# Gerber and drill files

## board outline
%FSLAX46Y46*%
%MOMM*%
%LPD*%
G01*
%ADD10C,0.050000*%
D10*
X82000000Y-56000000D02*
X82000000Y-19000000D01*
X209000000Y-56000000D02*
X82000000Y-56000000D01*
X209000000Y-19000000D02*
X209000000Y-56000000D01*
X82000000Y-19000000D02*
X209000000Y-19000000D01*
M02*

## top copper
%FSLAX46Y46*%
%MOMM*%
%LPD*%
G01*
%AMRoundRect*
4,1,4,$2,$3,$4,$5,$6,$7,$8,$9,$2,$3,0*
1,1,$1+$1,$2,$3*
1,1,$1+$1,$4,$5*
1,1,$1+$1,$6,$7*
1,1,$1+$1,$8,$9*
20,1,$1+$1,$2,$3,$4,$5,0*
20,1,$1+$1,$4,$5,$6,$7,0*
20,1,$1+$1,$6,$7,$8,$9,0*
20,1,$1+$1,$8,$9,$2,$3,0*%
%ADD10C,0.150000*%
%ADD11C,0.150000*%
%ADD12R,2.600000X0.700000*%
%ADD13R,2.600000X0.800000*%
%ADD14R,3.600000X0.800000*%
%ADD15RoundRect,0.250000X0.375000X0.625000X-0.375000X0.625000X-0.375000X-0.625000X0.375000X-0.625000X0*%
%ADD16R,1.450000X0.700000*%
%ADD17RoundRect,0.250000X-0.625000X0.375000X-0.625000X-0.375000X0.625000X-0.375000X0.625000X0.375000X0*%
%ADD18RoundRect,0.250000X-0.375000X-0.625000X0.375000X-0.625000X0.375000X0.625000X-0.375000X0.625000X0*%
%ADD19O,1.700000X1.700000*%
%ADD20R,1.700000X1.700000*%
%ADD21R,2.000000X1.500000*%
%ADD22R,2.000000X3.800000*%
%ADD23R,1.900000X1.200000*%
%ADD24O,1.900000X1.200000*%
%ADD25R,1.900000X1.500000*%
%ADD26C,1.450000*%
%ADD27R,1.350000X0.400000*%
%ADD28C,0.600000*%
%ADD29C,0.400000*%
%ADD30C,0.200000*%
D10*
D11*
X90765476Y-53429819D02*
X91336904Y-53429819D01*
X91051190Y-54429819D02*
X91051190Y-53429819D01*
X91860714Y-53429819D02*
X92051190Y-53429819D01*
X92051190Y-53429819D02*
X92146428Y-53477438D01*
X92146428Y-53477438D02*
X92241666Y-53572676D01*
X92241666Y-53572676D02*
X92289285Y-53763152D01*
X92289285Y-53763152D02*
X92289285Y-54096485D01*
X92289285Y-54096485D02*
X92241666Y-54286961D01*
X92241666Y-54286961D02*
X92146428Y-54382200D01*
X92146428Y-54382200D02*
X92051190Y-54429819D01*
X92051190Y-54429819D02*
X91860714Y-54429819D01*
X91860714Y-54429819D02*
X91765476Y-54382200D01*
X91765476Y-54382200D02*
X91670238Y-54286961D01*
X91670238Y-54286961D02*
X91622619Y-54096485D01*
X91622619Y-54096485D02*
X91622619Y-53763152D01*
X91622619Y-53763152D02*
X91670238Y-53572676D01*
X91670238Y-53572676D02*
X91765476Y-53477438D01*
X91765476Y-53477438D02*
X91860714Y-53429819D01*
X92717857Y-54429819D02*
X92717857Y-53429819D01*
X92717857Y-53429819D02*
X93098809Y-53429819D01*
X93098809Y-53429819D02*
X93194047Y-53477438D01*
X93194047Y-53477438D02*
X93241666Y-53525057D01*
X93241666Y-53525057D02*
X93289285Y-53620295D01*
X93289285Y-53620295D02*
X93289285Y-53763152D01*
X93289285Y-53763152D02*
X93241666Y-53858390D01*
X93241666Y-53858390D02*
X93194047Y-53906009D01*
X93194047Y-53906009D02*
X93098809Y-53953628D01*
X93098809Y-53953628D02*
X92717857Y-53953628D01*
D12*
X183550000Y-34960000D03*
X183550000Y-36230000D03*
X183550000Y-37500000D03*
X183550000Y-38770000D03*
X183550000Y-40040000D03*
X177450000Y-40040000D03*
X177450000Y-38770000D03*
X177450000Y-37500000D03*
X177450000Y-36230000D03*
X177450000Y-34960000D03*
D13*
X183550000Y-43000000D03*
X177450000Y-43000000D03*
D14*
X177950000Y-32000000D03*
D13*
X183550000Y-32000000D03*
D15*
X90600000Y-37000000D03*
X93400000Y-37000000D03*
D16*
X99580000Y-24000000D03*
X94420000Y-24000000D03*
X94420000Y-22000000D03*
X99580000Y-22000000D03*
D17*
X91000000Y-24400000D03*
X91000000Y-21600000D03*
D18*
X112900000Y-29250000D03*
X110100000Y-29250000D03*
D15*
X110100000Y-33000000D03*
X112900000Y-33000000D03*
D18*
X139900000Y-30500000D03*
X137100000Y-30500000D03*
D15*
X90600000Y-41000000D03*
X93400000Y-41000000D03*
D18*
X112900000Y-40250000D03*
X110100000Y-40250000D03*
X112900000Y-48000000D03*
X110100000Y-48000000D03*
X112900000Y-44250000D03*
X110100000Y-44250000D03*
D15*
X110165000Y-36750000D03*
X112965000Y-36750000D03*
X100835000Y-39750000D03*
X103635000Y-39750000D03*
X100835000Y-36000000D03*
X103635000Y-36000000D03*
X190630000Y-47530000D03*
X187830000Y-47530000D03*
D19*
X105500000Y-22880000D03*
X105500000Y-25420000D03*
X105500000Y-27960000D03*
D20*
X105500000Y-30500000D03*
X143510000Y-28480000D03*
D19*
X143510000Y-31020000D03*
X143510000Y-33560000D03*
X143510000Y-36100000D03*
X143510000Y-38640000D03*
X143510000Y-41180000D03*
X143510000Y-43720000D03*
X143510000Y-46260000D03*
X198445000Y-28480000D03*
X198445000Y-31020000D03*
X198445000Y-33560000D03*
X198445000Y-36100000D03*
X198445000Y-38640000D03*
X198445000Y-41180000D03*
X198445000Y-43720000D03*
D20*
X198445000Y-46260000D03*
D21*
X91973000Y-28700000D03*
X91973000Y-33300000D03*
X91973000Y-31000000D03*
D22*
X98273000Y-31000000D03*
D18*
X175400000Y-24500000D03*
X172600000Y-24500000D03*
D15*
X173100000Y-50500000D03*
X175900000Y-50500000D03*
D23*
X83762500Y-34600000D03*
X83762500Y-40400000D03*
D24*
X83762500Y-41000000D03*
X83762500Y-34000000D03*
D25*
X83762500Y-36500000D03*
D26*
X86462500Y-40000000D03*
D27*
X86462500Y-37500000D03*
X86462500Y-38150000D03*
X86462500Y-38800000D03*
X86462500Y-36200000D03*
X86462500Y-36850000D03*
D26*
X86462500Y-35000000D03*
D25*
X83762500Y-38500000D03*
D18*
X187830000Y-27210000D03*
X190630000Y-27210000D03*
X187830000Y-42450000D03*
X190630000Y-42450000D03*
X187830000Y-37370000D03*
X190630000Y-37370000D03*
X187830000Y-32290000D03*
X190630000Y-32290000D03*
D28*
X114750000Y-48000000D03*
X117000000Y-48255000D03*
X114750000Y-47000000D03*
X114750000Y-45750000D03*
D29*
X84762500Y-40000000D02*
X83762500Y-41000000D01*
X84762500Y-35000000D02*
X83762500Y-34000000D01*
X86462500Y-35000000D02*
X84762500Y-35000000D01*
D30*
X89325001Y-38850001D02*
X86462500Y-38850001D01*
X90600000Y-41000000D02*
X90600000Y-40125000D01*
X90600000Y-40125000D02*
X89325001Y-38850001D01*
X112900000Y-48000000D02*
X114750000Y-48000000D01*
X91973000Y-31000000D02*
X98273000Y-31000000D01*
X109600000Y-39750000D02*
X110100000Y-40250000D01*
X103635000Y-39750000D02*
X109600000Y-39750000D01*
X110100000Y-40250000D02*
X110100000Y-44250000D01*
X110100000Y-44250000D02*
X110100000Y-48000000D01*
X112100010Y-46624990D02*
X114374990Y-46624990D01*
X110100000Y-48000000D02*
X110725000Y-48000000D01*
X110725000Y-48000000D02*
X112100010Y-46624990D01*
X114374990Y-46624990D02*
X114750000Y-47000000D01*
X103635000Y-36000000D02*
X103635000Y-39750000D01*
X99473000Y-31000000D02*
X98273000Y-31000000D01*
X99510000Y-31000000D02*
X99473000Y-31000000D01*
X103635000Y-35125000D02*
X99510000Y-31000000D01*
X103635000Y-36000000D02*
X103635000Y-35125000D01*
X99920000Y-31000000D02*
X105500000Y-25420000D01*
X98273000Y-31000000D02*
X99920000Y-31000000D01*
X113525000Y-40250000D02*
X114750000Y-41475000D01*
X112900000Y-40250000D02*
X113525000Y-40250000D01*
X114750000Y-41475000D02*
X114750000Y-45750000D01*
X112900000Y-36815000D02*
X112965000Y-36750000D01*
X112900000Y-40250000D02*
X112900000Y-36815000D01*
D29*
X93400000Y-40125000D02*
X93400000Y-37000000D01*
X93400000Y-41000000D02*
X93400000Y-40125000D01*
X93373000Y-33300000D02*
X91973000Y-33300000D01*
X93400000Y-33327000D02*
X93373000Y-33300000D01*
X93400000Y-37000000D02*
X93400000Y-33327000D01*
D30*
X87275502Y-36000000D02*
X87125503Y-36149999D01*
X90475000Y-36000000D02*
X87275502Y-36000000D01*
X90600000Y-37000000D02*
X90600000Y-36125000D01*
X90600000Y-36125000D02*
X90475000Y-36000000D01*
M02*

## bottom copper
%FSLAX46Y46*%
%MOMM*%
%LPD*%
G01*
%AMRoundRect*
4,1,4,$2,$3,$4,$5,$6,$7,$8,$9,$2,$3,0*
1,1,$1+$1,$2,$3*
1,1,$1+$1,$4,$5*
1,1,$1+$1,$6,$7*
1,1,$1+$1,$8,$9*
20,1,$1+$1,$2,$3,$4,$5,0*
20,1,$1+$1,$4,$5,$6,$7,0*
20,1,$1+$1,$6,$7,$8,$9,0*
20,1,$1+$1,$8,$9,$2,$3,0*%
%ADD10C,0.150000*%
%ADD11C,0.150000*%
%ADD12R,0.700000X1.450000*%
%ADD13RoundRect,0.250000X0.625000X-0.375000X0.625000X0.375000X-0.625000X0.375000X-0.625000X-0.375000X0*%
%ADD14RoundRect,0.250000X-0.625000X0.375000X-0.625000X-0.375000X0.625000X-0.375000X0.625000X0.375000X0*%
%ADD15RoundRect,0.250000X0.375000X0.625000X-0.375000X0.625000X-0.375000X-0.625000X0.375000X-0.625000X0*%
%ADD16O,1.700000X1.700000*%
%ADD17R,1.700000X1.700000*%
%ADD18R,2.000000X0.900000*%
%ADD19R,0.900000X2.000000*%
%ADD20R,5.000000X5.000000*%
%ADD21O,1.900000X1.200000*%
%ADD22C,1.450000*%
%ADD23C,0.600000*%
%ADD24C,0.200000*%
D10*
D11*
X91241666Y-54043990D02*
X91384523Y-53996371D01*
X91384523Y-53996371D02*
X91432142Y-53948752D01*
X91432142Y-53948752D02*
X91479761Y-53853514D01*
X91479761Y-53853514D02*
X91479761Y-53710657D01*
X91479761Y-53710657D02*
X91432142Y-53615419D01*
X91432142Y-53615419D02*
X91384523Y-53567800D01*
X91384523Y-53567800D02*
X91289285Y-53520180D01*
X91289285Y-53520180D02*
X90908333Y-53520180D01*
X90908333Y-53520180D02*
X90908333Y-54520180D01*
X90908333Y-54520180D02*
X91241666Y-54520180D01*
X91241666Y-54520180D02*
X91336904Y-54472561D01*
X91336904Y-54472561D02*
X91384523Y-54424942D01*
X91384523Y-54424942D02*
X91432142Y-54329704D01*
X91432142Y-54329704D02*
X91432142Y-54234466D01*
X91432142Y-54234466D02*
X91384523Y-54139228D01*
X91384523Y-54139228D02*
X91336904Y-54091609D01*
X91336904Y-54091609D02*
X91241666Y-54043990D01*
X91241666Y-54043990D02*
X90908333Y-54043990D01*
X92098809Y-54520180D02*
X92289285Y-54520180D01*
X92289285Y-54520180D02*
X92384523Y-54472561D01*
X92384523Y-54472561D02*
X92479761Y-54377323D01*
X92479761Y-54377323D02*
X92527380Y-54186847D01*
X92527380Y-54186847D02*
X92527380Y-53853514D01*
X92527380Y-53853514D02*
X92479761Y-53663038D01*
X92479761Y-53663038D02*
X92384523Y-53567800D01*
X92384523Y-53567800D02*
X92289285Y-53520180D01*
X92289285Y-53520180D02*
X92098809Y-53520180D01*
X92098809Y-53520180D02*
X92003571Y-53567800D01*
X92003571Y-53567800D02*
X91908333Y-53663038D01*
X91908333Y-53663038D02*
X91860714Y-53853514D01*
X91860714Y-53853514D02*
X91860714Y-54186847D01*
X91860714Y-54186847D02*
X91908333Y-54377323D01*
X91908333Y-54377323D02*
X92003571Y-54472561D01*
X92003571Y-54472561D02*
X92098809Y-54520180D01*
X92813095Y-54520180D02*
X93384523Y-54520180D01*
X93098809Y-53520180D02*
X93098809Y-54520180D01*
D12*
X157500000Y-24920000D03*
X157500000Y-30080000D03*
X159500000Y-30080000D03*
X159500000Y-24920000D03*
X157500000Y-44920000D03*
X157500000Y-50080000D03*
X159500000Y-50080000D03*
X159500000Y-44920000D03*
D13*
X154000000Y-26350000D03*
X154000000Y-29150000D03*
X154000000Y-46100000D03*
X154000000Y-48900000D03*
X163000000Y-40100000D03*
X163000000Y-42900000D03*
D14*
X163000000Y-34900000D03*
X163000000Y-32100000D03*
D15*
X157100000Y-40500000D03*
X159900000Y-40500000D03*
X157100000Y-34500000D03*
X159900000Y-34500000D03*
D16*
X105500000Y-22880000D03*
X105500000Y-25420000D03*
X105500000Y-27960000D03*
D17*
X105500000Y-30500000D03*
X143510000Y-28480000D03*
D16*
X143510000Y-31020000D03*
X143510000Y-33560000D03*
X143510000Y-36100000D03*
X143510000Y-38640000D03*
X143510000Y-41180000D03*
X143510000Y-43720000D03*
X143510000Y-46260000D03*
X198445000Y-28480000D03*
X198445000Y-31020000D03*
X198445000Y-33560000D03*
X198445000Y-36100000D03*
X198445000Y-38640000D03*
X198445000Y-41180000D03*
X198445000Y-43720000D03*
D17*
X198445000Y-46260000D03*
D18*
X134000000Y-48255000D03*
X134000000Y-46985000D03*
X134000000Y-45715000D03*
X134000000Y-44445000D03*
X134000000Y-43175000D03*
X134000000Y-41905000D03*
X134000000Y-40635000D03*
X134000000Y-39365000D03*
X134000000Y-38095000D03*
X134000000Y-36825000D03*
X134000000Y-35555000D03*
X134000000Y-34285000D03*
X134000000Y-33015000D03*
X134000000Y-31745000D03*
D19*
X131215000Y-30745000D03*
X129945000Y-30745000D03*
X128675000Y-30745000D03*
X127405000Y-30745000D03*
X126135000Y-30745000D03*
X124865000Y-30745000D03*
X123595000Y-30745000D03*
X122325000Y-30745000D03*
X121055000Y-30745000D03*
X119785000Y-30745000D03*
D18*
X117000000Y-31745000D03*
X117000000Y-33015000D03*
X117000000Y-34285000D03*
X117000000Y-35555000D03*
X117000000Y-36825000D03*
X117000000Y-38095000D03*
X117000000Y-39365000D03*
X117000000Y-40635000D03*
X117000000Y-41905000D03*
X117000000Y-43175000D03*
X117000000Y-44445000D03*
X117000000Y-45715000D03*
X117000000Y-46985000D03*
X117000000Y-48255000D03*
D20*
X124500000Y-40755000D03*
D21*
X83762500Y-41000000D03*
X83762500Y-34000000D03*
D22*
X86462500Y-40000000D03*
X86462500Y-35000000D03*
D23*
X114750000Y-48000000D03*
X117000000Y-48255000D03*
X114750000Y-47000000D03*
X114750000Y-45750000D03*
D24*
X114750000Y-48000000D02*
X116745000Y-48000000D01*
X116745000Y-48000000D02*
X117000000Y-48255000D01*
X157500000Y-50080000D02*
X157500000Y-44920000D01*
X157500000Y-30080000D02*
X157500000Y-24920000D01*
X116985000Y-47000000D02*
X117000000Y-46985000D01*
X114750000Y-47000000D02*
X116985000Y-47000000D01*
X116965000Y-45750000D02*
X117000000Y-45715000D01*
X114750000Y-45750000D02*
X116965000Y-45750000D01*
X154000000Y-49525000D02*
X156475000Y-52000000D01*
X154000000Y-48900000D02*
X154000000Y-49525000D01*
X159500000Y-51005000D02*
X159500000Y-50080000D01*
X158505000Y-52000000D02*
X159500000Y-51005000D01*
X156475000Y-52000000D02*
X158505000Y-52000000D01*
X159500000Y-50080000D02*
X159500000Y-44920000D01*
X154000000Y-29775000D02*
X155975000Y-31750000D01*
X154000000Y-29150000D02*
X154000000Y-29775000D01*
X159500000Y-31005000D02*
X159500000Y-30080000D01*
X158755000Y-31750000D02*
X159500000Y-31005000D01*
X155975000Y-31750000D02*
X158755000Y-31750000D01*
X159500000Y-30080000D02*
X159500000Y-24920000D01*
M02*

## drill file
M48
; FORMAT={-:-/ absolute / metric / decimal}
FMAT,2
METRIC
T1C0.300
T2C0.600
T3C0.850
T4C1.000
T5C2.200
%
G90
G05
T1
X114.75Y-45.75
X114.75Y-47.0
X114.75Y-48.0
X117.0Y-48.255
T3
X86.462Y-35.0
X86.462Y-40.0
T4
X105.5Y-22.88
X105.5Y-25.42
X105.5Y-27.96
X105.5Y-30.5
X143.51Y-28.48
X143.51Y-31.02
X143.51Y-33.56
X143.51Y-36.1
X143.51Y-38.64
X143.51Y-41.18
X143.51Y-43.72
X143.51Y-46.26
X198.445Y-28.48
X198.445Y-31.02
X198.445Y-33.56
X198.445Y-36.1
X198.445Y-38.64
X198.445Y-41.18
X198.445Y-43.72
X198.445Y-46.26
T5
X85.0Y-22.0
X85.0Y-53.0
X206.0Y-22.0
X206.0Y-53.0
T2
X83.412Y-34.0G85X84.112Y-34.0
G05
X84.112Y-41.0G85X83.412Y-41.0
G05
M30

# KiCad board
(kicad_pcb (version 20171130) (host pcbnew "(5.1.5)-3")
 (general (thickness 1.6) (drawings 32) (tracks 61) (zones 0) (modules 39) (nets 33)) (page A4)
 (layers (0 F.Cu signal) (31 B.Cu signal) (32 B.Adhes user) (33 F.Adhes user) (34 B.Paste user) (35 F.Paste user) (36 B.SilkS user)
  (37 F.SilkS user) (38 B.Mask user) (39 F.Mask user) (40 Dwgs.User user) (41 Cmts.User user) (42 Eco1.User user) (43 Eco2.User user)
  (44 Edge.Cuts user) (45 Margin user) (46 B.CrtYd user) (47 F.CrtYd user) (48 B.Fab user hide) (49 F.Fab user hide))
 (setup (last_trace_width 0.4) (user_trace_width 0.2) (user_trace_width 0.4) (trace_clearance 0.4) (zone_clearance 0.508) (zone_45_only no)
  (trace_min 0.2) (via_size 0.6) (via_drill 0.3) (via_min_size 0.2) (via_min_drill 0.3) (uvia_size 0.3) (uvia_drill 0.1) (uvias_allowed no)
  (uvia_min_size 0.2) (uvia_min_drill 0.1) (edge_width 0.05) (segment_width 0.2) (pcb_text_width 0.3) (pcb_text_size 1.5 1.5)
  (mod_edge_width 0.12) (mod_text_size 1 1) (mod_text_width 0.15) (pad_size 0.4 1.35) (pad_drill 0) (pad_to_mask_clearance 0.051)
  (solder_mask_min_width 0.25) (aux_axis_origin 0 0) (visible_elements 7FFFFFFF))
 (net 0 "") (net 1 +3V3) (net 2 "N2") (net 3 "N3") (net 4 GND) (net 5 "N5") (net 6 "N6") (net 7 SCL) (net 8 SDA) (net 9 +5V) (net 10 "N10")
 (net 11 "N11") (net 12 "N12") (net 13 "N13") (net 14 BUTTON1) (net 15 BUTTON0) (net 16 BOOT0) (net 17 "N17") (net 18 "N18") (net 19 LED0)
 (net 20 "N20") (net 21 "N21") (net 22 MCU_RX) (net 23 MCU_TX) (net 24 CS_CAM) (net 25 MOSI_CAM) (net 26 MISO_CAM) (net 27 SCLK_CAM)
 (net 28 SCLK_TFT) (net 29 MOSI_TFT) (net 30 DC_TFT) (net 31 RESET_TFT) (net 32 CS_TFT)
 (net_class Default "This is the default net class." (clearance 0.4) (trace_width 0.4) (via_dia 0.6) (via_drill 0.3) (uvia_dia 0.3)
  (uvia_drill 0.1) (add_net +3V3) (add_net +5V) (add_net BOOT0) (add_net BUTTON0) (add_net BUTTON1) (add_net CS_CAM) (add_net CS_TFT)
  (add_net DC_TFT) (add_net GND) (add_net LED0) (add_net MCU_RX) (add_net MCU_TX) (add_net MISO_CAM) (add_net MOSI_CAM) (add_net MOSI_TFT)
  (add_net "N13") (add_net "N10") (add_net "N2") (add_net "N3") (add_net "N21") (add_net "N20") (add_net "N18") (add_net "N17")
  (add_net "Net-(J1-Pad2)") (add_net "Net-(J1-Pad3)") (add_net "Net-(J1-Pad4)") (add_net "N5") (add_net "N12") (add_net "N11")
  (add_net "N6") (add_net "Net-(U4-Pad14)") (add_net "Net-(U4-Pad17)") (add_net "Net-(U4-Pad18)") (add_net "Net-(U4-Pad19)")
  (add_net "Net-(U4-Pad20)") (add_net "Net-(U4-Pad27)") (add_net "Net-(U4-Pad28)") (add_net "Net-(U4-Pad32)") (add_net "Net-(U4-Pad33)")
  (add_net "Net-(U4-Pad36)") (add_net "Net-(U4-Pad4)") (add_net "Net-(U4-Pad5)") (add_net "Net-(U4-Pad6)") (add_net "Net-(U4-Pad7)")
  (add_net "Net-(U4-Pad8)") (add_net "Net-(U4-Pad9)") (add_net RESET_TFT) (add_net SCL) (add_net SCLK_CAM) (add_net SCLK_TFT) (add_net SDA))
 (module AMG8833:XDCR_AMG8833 (layer F.Cu) (at 180.5 37.5 270)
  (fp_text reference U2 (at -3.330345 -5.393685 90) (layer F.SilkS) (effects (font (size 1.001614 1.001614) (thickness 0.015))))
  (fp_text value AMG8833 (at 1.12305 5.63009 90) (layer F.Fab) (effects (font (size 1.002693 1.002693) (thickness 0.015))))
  (pad 13 smd rect (at -2.54 -3.05 270) (size 0.7 2.6) (layers F.Cu F.Paste F.Mask) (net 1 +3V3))
  (pad 12 smd rect (at -1.27 -3.05 270) (size 0.7 2.6) (layers F.Cu F.Paste F.Mask) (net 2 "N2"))
  (pad 11 smd rect (at 0 -3.05 270) (size 0.7 2.6) (layers F.Cu F.Paste F.Mask))
  (pad 10 smd rect (at 1.27 -3.05 270) (size 0.7 2.6) (layers F.Cu F.Paste F.Mask) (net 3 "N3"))
  (pad 9 smd rect (at 2.54 -3.05 270) (size 0.7 2.6) (layers F.Cu F.Paste F.Mask) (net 1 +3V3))
  (pad 6 smd rect (at 2.54 3.05 270) (size 0.7 2.6) (layers F.Cu F.Paste F.Mask) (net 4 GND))
  (pad 5 smd rect (at 1.27 3.05 270) (size 0.7 2.6) (layers F.Cu F.Paste F.Mask) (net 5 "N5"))
  (pad 4 smd rect (at 0 3.05 270) (size 0.7 2.6) (layers F.Cu F.Paste F.Mask) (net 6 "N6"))
  (pad 3 smd rect (at -1.27 3.05 270) (size 0.7 2.6) (layers F.Cu F.Paste F.Mask) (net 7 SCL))
  (pad 2 smd rect (at -2.54 3.05 270) (size 0.7 2.6) (layers F.Cu F.Paste F.Mask) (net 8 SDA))
  (pad 8 smd rect (at 5.5 -3.05 270) (size 0.8 2.6) (layers F.Cu F.Paste F.Mask))
  (pad 7 smd rect (at 5.5 3.05 270) (size 0.8 2.6) (layers F.Cu F.Paste F.Mask))
  (pad 1 smd rect (at -5.5 2.55 270) (size 0.8 3.6) (layers F.Cu F.Paste F.Mask))
  (pad 14 smd rect (at -5.5 -3.05 270) (size 0.8 2.6) (layers F.Cu F.Paste F.Mask)))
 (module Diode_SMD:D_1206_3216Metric (layer F.Cu) (at 92 37 180)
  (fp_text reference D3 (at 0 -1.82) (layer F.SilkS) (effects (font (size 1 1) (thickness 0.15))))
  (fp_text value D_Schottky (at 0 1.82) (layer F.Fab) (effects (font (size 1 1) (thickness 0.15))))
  (pad 2 smd roundrect (at 1.4 0 180) (size 1.25 1.75) (layers F.Cu F.Paste F.Mask) (roundrect_rratio 0.2) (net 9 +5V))
  (pad 1 smd roundrect (at -1.4 0 180) (size 1.25 1.75) (layers F.Cu F.Paste F.Mask) (roundrect_rratio 0.2) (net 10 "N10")))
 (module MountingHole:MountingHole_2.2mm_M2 (layer F.Cu) (at 206 22)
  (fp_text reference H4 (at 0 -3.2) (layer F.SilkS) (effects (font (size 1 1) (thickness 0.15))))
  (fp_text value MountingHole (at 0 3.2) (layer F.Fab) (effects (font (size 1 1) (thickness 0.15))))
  (pad 1 np_thru_hole circle (at 0 0) (size 2.2 2.2) (drill 2.2) (layers *.Cu *.Mask)))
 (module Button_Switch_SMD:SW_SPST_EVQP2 (layer B.Cu) (at 158.5 27.5 90)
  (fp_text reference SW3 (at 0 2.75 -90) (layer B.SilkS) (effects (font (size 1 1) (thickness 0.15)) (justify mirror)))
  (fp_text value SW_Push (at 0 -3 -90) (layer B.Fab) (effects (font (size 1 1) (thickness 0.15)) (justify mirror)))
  (pad 2 smd rect (at 2.58 -1 90) (size 1.45 0.7) (layers B.Cu B.Paste B.Mask) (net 4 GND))
  (pad 2 smd rect (at -2.58 -1 90) (size 1.45 0.7) (layers B.Cu B.Paste B.Mask) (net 4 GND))
  (pad 1 smd rect (at -2.58 1 90) (size 1.45 0.7) (layers B.Cu B.Paste B.Mask) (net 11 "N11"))
  (pad 1 smd rect (at 2.58 1 90) (size 1.45 0.7) (layers B.Cu B.Paste B.Mask) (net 11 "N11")))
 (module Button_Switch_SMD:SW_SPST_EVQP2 (layer B.Cu) (at 158.5 47.5 90)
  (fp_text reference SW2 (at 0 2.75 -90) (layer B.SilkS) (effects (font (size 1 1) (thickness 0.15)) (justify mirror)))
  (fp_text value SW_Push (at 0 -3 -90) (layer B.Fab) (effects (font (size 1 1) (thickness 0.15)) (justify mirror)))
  (pad 2 smd rect (at 2.58 -1 90) (size 1.45 0.7) (layers B.Cu B.Paste B.Mask) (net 4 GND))
  (pad 2 smd rect (at -2.58 -1 90) (size 1.45 0.7) (layers B.Cu B.Paste B.Mask) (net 4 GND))
  (pad 1 smd rect (at -2.58 1 90) (size 1.45 0.7) (layers B.Cu B.Paste B.Mask) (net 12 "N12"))
  (pad 1 smd rect (at 2.58 1 90) (size 1.45 0.7) (layers B.Cu B.Paste B.Mask) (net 12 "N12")))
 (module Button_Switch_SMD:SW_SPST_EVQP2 (layer F.Cu) (at 97 23)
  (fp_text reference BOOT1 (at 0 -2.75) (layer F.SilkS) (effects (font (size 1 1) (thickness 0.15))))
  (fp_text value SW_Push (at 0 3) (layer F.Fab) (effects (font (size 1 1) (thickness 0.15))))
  (pad 2 smd rect (at 2.58 1) (size 1.45 0.7) (layers F.Cu F.Paste F.Mask) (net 4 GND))
  (pad 2 smd rect (at -2.58 1) (size 1.45 0.7) (layers F.Cu F.Paste F.Mask) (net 4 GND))
  (pad 1 smd rect (at -2.58 -1) (size 1.45 0.7) (layers F.Cu F.Paste F.Mask) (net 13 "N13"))
  (pad 1 smd rect (at 2.58 -1) (size 1.45 0.7) (layers F.Cu F.Paste F.Mask) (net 13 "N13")))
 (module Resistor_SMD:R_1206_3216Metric (layer B.Cu) (at 154 27.75 90)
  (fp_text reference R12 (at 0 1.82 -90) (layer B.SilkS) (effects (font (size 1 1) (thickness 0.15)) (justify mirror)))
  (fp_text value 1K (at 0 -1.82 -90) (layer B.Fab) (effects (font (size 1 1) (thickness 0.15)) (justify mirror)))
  (pad 2 smd roundrect (at 1.4 0 90) (size 1.25 1.75) (layers B.Cu B.Paste B.Mask) (roundrect_rratio 0.2) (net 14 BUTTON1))
  (pad 1 smd roundrect (at -1.4 0 90) (size 1.25 1.75) (layers B.Cu B.Paste B.Mask) (roundrect_rratio 0.2) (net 11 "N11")))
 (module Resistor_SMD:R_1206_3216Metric (layer B.Cu) (at 154 47.5 90)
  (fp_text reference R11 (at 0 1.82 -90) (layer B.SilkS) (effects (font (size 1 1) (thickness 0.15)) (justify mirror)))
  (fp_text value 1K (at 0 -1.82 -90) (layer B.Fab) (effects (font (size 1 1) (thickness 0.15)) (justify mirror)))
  (pad 2 smd roundrect (at 1.4 0 90) (size 1.25 1.75) (layers B.Cu B.Paste B.Mask) (roundrect_rratio 0.2) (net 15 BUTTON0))
  (pad 1 smd roundrect (at -1.4 0 90) (size 1.25 1.75) (layers B.Cu B.Paste B.Mask) (roundrect_rratio 0.2) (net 12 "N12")))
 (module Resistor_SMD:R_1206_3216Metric (layer F.Cu) (at 91 23 270)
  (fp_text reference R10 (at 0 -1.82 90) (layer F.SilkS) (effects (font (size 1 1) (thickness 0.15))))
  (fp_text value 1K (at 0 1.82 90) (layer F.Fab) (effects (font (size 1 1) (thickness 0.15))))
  (pad 2 smd roundrect (at 1.4 0 270) (size 1.25 1.75) (layers F.Cu F.Paste F.Mask) (roundrect_rratio 0.2) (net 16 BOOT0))
  (pad 1 smd roundrect (at -1.4 0 270) (size 1.25 1.75) (layers F.Cu F.Paste F.Mask) (roundrect_rratio 0.2) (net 13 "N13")))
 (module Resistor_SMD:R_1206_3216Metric (layer F.Cu) (at 111.5 29.25)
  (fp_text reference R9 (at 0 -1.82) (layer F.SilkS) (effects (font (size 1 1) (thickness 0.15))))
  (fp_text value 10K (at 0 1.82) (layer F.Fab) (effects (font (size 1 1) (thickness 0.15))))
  (pad 2 smd roundrect (at 1.4 0) (size 1.25 1.75) (layers F.Cu F.Paste F.Mask) (roundrect_rratio 0.2) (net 1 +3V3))
  (pad 1 smd roundrect (at -1.4 0) (size 1.25 1.75) (layers F.Cu F.Paste F.Mask) (roundrect_rratio 0.2) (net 14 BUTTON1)))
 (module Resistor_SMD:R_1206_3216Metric (layer F.Cu) (at 111.5 33 180)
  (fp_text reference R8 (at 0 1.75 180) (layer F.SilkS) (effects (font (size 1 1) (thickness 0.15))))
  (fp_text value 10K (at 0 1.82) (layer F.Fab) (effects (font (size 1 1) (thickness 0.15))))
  (pad 2 smd roundrect (at 1.4 0 180) (size 1.25 1.75) (layers F.Cu F.Paste F.Mask) (roundrect_rratio 0.2) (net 1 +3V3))
  (pad 1 smd roundrect (at -1.4 0 180) (size 1.25 1.75) (layers F.Cu F.Paste F.Mask) (roundrect_rratio 0.2) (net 15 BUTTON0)))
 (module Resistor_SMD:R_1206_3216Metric (layer F.Cu) (at 138.5 30.5)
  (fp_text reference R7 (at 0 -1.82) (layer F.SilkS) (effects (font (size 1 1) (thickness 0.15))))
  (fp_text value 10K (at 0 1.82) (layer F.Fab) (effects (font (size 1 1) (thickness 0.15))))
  (pad 2 smd roundrect (at 1.4 0) (size 1.25 1.75) (layers F.Cu F.Paste F.Mask) (roundrect_rratio 0.2) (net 1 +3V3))
  (pad 1 smd roundrect (at -1.4 0) (size 1.25 1.75) (layers F.Cu F.Paste F.Mask) (roundrect_rratio 0.2) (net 16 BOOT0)))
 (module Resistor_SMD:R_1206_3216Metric (layer B.Cu) (at 163 41.5 90)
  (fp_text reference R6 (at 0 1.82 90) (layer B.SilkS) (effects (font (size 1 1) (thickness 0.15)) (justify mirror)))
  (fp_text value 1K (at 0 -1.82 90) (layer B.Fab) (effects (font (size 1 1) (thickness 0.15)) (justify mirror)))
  (pad 2 smd roundrect (at 1.4 0 90) (size 1.25 1.75) (layers B.Cu B.Paste B.Mask) (roundrect_rratio 0.2) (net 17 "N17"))
  (pad 1 smd roundrect (at -1.4 0 90) (size 1.25 1.75) (layers B.Cu B.Paste B.Mask) (roundrect_rratio 0.2) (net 4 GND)))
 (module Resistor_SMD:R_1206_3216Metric (layer B.Cu) (at 163 33.5 270)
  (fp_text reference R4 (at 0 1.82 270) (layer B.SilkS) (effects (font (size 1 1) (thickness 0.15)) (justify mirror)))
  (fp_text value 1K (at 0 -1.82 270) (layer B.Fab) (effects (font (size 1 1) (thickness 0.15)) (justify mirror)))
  (pad 2 smd roundrect (at 1.4 0 270) (size 1.25 1.75) (layers B.Cu B.Paste B.Mask) (roundrect_rratio 0.2) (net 4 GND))
  (pad 1 smd roundrect (at -1.4 0 270) (size 1.25 1.75) (layers B.Cu B.Paste B.Mask) (roundrect_rratio 0.2) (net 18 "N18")))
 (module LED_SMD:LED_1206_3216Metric (layer B.Cu) (at 158.5 40.5 180)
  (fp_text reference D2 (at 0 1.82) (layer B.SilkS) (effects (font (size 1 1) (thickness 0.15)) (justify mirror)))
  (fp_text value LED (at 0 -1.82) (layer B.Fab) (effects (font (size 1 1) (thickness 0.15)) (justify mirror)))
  (pad 2 smd roundrect (at 1.4 0 180) (size 1.25 1.75) (layers B.Cu B.Paste B.Mask) (roundrect_rratio 0.2) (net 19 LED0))
  (pad 1 smd roundrect (at -1.4 0 180) (size 1.25 1.75) (layers B.Cu B.Paste B.Mask) (roundrect_rratio 0.2) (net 17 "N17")))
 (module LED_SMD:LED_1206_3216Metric (layer B.Cu) (at 158.5 34.5 180)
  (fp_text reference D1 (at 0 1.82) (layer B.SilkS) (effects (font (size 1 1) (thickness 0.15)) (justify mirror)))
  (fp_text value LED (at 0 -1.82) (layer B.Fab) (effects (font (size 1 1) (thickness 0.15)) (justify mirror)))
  (pad 2 smd roundrect (at 1.4 0 180) (size 1.25 1.75) (layers B.Cu B.Paste B.Mask) (roundrect_rratio 0.2) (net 1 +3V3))
  (pad 1 smd roundrect (at -1.4 0 180) (size 1.25 1.75) (layers B.Cu B.Paste B.Mask) (roundrect_rratio 0.2) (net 18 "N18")))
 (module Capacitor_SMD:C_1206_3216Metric (layer F.Cu) (at 92 41 180)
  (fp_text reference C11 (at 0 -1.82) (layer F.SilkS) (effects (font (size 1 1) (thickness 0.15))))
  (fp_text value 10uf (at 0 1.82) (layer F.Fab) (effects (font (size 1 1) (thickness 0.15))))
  (pad 2 smd roundrect (at 1.4 0 180) (size 1.25 1.75) (layers F.Cu F.Paste F.Mask) (roundrect_rratio 0.2) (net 4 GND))
  (pad 1 smd roundrect (at -1.4 0 180) (size 1.25 1.75) (layers F.Cu F.Paste F.Mask) (roundrect_rratio 0.2) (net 10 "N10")))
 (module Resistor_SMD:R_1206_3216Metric (layer F.Cu) (at 111.5 40.25)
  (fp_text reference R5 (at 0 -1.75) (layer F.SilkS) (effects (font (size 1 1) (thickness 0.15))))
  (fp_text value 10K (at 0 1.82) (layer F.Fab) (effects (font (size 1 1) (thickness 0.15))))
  (pad 2 smd roundrect (at 1.4 0) (size 1.25 1.75) (layers F.Cu F.Paste F.Mask) (roundrect_rratio 0.2) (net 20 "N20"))
  (pad 1 smd roundrect (at -1.4 0) (size 1.25 1.75) (layers F.Cu F.Paste F.Mask) (roundrect_rratio 0.2) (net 1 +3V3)))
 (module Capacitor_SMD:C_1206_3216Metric (layer F.Cu) (at 111.5 48)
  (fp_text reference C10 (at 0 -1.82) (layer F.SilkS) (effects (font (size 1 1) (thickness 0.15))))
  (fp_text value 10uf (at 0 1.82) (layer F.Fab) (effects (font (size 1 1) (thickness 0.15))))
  (pad 2 smd roundrect (at 1.4 0) (size 1.25 1.75) (layers F.Cu F.Paste F.Mask) (roundrect_rratio 0.2) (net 4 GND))
  (pad 1 smd roundrect (at -1.4 0) (size 1.25 1.75) (layers F.Cu F.Paste F.Mask) (roundrect_rratio 0.2) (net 1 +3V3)))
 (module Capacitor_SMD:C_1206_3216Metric (layer F.Cu) (at 111.5 44.25)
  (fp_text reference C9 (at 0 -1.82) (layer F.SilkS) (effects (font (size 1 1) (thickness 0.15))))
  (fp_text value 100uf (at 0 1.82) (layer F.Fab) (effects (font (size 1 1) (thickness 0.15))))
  (pad 2 smd roundrect (at 1.4 0) (size 1.25 1.75) (layers F.Cu F.Paste F.Mask) (roundrect_rratio 0.2) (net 4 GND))
  (pad 1 smd roundrect (at -1.4 0) (size 1.25 1.75) (layers F.Cu F.Paste F.Mask) (roundrect_rratio 0.2) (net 1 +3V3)))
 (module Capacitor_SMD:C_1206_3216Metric (layer F.Cu) (at 111.565 36.75 180)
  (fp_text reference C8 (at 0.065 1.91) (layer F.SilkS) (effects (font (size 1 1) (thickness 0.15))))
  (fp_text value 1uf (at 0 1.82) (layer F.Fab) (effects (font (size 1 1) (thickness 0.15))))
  (pad 2 smd roundrect (at 1.4 0 180) (size 1.25 1.75) (layers F.Cu F.Paste F.Mask) (roundrect_rratio 0.2) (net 4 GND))
  (pad 1 smd roundrect (at -1.4 0 180) (size 1.25 1.75) (layers F.Cu F.Paste F.Mask) (roundrect_rratio 0.2) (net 20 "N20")))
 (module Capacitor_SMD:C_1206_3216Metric (layer F.Cu) (at 102.235 39.75 180)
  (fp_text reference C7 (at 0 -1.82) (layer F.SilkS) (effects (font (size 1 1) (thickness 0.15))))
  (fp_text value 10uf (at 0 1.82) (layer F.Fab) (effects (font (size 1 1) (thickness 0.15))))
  (pad 2 smd roundrect (at 1.4 0 180) (size 1.25 1.75) (layers F.Cu F.Paste F.Mask) (roundrect_rratio 0.2) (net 4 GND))
  (pad 1 smd roundrect (at -1.4 0 180) (size 1.25 1.75) (layers F.Cu F.Paste F.Mask) (roundrect_rratio 0.2) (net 1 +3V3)))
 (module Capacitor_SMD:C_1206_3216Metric (layer F.Cu) (at 102.235 36 180)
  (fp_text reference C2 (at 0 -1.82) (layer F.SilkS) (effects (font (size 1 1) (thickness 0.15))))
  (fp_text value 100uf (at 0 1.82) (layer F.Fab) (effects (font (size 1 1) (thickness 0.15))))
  (pad 2 smd roundrect (at 1.4 0 180) (size 1.25 1.75) (layers F.Cu F.Paste F.Mask) (roundrect_rratio 0.2) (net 4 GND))
  (pad 1 smd roundrect (at -1.4 0 180) (size 1.25 1.75) (layers F.Cu F.Paste F.Mask) (roundrect_rratio 0.2) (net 1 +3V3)))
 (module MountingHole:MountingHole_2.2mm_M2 (layer F.Cu) (at 206 53)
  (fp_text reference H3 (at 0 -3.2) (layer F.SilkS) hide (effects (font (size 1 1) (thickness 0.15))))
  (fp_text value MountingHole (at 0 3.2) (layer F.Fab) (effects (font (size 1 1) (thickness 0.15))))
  (pad 1 np_thru_hole circle (at 0 0) (size 2.2 2.2) (drill 2.2) (layers *.Cu *.Mask)))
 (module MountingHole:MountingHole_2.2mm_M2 (layer F.Cu) (at 85 53)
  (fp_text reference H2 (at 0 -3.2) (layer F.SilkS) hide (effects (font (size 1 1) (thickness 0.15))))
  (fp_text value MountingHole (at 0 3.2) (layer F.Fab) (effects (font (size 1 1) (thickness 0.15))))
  (pad 1 np_thru_hole circle (at 0 0) (size 2.2 2.2) (drill 2.2) (layers *.Cu *.Mask)))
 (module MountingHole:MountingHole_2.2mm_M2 (layer F.Cu) (at 85 22)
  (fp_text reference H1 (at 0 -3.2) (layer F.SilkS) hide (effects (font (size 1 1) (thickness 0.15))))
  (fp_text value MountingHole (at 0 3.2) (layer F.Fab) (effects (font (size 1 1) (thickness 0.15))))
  (pad 1 np_thru_hole circle (at 0 0) (size 2.2 2.2) (drill 2.2) (layers *.Cu *.Mask)))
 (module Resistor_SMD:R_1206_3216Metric (layer F.Cu) (at 189.23 47.53 180)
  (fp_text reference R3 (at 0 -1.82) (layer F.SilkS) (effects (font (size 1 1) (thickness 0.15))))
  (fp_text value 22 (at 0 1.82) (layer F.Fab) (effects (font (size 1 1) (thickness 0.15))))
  (pad 1 smd roundrect (at -1.4 0 180) (size 1.25 1.75) (layers F.Cu F.Paste F.Mask) (roundrect_rratio 0.2) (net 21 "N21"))
  (pad 2 smd roundrect (at 1.4 0 180) (size 1.25 1.75) (layers F.Cu F.Paste F.Mask) (roundrect_rratio 0.2) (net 4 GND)))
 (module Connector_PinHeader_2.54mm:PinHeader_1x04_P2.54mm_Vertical (layer F.Cu) (at 105.5 30.5 180)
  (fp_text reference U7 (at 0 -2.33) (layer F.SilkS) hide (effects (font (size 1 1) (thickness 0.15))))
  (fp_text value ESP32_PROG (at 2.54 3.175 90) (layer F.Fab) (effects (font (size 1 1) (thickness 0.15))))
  (pad 4 thru_hole oval (at 0 7.62 180) (size 1.7 1.7) (drill 1) (layers *.Cu *.Mask) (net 4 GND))
  (pad 3 thru_hole oval (at 0 5.08 180) (size 1.7 1.7) (drill 1) (layers *.Cu *.Mask) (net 1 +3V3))
  (pad 2 thru_hole oval (at 0 2.54 180) (size 1.7 1.7) (drill 1) (layers *.Cu *.Mask) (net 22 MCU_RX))
  (pad 1 thru_hole rect (at 0 0 180) (size 1.7 1.7) (drill 1) (layers *.Cu *.Mask) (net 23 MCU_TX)))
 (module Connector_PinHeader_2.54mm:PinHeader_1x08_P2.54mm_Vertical (layer F.Cu) (at 143.51 28.48)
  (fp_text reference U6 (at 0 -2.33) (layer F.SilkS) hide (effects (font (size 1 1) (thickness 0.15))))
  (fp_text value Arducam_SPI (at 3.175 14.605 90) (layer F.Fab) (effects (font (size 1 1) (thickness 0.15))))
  (pad 1 thru_hole rect (at 0 0) (size 1.7 1.7) (drill 1) (layers *.Cu *.Mask) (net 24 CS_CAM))
  (pad 2 thru_hole oval (at 0 2.54) (size 1.7 1.7) (drill 1) (layers *.Cu *.Mask) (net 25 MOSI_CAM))
  (pad 3 thru_hole oval (at 0 5.08) (size 1.7 1.7) (drill 1) (layers *.Cu *.Mask) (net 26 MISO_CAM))
  (pad 4 thru_hole oval (at 0 7.62) (size 1.7 1.7) (drill 1) (layers *.Cu *.Mask) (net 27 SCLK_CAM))
  (pad 5 thru_hole oval (at 0 10.16) (size 1.7 1.7) (drill 1) (layers *.Cu *.Mask) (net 4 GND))
  (pad 6 thru_hole oval (at 0 12.7) (size 1.7 1.7) (drill 1) (layers *.Cu *.Mask) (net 1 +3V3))
  (pad 7 thru_hole oval (at 0 15.24) (size 1.7 1.7) (drill 1) (layers *.Cu *.Mask) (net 8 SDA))
  (pad 8 thru_hole oval (at 0 17.78) (size 1.7 1.7) (drill 1) (layers *.Cu *.Mask) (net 7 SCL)))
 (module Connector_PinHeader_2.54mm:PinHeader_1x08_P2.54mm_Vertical (layer B.Cu) (at 198.445 46.26)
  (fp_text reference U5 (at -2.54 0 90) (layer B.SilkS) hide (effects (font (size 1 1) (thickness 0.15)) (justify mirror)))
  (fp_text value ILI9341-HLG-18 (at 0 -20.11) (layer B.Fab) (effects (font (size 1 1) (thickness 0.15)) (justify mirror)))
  (pad 8 thru_hole oval (at 0 -17.78) (size 1.7 1.7) (drill 1) (layers *.Cu *.Mask) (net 1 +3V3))
  (pad 7 thru_hole oval (at 0 -15.24) (size 1.7 1.7) (drill 1) (layers *.Cu *.Mask) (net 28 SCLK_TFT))
  (pad 6 thru_hole oval (at 0 -12.7) (size 1.7 1.7) (drill 1) (layers *.Cu *.Mask) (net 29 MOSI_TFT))
  (pad 5 thru_hole oval (at 0 -10.16) (size 1.7 1.7) (drill 1) (layers *.Cu *.Mask) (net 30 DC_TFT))
  (pad 4 thru_hole oval (at 0 -7.62) (size 1.7 1.7) (drill 1) (layers *.Cu *.Mask) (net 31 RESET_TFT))
  (pad 3 thru_hole oval (at 0 -5.08) (size 1.7 1.7) (drill 1) (layers *.Cu *.Mask) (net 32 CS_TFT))
  (pad 2 thru_hole oval (at 0 -2.54) (size 1.7 1.7) (drill 1) (layers *.Cu *.Mask) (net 4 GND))
  (pad 1 thru_hole rect (at 0 0) (size 1.7 1.7) (drill 1) (layers *.Cu *.Mask) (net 1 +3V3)))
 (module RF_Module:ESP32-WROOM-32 (layer B.Cu) (at 125.5 40)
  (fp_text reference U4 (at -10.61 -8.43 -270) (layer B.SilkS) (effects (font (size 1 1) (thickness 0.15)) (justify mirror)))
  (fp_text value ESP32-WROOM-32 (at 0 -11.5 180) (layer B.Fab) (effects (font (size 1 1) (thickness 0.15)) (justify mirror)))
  (pad 38 smd rect (at 8.5 8.255) (size 2 0.9) (layers B.Cu B.Paste B.Mask) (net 4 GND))
  (pad 37 smd rect (at 8.5 6.985) (size 2 0.9) (layers B.Cu B.Paste B.Mask) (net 25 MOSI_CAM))
  (pad 36 smd rect (at 8.5 5.715) (size 2 0.9) (layers B.Cu B.Paste B.Mask))
  (pad 35 smd rect (at 8.5 4.445) (size 2 0.9) (layers B.Cu B.Paste B.Mask) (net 23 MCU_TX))
  (pad 34 smd rect (at 8.5 3.175) (size 2 0.9) (layers B.Cu B.Paste B.Mask) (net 22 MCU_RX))
  (pad 33 smd rect (at 8.5 1.905) (size 2 0.9) (layers B.Cu B.Paste B.Mask))
  (pad 32 smd rect (at 8.5 0.635) (size 2 0.9) (layers B.Cu B.Paste B.Mask))
  (pad 31 smd rect (at 8.5 -0.635) (size 2 0.9) (layers B.Cu B.Paste B.Mask) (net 26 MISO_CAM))
  (pad 30 smd rect (at 8.5 -1.905) (size 2 0.9) (layers B.Cu B.Paste B.Mask) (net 27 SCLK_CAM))
  (pad 29 smd rect (at 8.5 -3.175) (size 2 0.9) (layers B.Cu B.Paste B.Mask) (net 24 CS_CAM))
  (pad 28 smd rect (at 8.5 -4.445) (size 2 0.9) (layers B.Cu B.Paste B.Mask))
  (pad 27 smd rect (at 8.5 -5.715) (size 2 0.9) (layers B.Cu B.Paste B.Mask))
  (pad 26 smd rect (at 8.5 -6.985) (size 2 0.9) (layers B.Cu B.Paste B.Mask) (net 31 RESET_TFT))
  (pad 25 smd rect (at 8.5 -8.255) (size 2 0.9) (layers B.Cu B.Paste B.Mask) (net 16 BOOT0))
  (pad 24 smd rect (at 5.715 -9.255 270) (size 2 0.9) (layers B.Cu B.Paste B.Mask) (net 30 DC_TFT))
  (pad 23 smd rect (at 4.445 -9.255 270) (size 2 0.9) (layers B.Cu B.Paste B.Mask) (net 32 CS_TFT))
  (pad 22 smd rect (at 3.175 -9.255 270) (size 2 0.9) (layers B.Cu B.Paste B.Mask) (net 7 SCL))
  (pad 21 smd rect (at 1.905 -9.255 270) (size 2 0.9) (layers B.Cu B.Paste B.Mask) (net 8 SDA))
  (pad 20 smd rect (at 0.635 -9.255 270) (size 2 0.9) (layers B.Cu B.Paste B.Mask))
  (pad 19 smd rect (at -0.635 -9.255 270) (size 2 0.9) (layers B.Cu B.Paste B.Mask))
  (pad 18 smd rect (at -1.905 -9.255 270) (size 2 0.9) (layers B.Cu B.Paste B.Mask))
  (pad 17 smd rect (at -3.175 -9.255 270) (size 2 0.9) (layers B.Cu B.Paste B.Mask))
  (pad 16 smd rect (at -4.445 -9.255 270) (size 2 0.9) (layers B.Cu B.Paste B.Mask) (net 29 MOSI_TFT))
  (pad 15 smd rect (at -5.715 -9.255 270) (size 2 0.9) (layers B.Cu B.Paste B.Mask) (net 4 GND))
  (pad 14 smd rect (at -8.5 -8.255) (size 2 0.9) (layers B.Cu B.Paste B.Mask))
  (pad 13 smd rect (at -8.5 -6.985) (size 2 0.9) (layers B.Cu B.Paste B.Mask) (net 28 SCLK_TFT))
  (pad 12 smd rect (at -8.5 -5.715) (size 2 0.9) (layers B.Cu B.Paste B.Mask) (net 19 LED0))
  (pad 11 smd rect (at -8.5 -4.445) (size 2 0.9) (layers B.Cu B.Paste B.Mask) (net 14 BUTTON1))
  (pad 10 smd rect (at -8.5 -3.175) (size 2 0.9) (layers B.Cu B.Paste B.Mask) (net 15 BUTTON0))
  (pad 9 smd rect (at -8.5 -1.905) (size 2 0.9) (layers B.Cu B.Paste B.Mask))
  (pad 8 smd rect (at -8.5 -0.635) (size 2 0.9) (layers B.Cu B.Paste B.Mask))
  (pad 7 smd rect (at -8.5 0.635) (size 2 0.9) (layers B.Cu B.Paste B.Mask))
  (pad 6 smd rect (at -8.5 1.905) (size 2 0.9) (layers B.Cu B.Paste B.Mask))
  (pad 5 smd rect (at -8.5 3.175) (size 2 0.9) (layers B.Cu B.Paste B.Mask))
  (pad 4 smd rect (at -8.5 4.445) (size 2 0.9) (layers B.Cu B.Paste B.Mask))
  (pad 3 smd rect (at -8.5 5.715) (size 2 0.9) (layers B.Cu B.Paste B.Mask) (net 20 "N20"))
  (pad 2 smd rect (at -8.5 6.985) (size 2 0.9) (layers B.Cu B.Paste B.Mask) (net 1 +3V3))
  (pad 1 smd rect (at -8.5 8.255) (size 2 0.9) (layers B.Cu B.Paste B.Mask) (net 4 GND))
  (pad 39 smd rect (at -1 0.755) (size 5 5) (layers B.Cu B.Paste B.Mask) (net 4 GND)))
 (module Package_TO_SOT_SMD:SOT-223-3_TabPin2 (layer F.Cu) (at 95.123 31)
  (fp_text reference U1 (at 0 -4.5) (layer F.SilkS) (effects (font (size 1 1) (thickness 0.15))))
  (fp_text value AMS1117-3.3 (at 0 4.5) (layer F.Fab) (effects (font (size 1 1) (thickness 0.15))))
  (pad 1 smd rect (at -3.15 -2.3) (size 2 1.5) (layers F.Cu F.Paste F.Mask) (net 4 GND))
  (pad 3 smd rect (at -3.15 2.3) (size 2 1.5) (layers F.Cu F.Paste F.Mask) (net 10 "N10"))
  (pad 2 smd rect (at -3.15 0) (size 2 1.5) (layers F.Cu F.Paste F.Mask) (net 1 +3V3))
  (pad 2 smd rect (at 3.15 0) (size 2 3.8) (layers F.Cu F.Paste F.Mask) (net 1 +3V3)))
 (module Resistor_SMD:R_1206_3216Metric (layer F.Cu) (at 174 24.5)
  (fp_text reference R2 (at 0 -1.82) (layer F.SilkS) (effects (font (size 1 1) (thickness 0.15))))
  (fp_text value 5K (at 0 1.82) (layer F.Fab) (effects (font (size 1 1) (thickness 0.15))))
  (pad 2 smd roundrect (at 1.4 0) (size 1.25 1.75) (layers F.Cu F.Paste F.Mask) (roundrect_rratio 0.2) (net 1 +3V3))
  (pad 1 smd roundrect (at -1.4 0) (size 1.25 1.75) (layers F.Cu F.Paste F.Mask) (roundrect_rratio 0.2) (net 6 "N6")))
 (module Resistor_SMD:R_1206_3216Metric (layer F.Cu) (at 174.5 50.5 180)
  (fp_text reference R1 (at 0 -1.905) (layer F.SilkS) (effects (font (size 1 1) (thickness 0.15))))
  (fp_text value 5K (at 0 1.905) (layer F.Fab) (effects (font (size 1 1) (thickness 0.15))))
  (pad 2 smd roundrect (at 1.4 0 180) (size 1.25 1.75) (layers F.Cu F.Paste F.Mask) (roundrect_rratio 0.2) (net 5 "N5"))
  (pad 1 smd roundrect (at -1.4 0 180) (size 1.25 1.75) (layers F.Cu F.Paste F.Mask) (roundrect_rratio 0.2) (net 1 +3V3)))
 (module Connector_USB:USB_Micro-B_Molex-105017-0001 (layer F.Cu) (at 85 37.5 270) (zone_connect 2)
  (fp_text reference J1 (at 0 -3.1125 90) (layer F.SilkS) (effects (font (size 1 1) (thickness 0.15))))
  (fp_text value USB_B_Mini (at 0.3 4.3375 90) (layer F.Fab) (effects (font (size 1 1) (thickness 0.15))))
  (pad 6 smd rect (at -2.9 1.2375 270) (size 1.2 1.9) (layers F.Cu F.Mask) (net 4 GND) (zone_connect 2))
  (pad 6 smd rect (at 2.9 1.2375 270) (size 1.2 1.9) (layers F.Cu F.Mask) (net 4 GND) (zone_connect 2))
  (pad 6 thru_hole oval (at 3.5 1.2375 270) (size 1.2 1.9) (drill oval 0.6 1.3) (layers *.Cu *.Mask) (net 4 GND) (zone_connect 2))
  (pad 6 thru_hole oval (at -3.5 1.2375 90) (size 1.2 1.9) (drill oval 0.6 1.3) (layers *.Cu *.Mask) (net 4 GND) (zone_connect 2))
  (pad 6 smd rect (at -1 1.2375 270) (size 1.5 1.9) (layers F.Cu F.Paste F.Mask) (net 4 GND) (zone_connect 2))
  (pad 6 thru_hole circle (at 2.5 -1.4625 270) (size 1.45 1.45) (drill 0.85) (layers *.Cu *.Mask) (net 4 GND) (zone_connect 2))
  (pad 3 smd rect (at 0 -1.4625 270) (size 0.4 1.35) (layers F.Cu F.Paste F.Mask) (zone_connect 2))
  (pad 4 smd rect (at 0.65 -1.4625 270) (size 0.4 1.35) (layers F.Cu F.Paste F.Mask) (zone_connect 2))
  (pad 5 smd rect (at 1.3 -1.4625 270) (size 0.4 1.35) (layers F.Cu F.Paste F.Mask) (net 4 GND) (zone_connect 2))
  (pad 1 smd rect (at -1.3 -1.4625 270) (size 0.4 1.35) (layers F.Cu F.Paste F.Mask) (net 9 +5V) (zone_connect 2))
  (pad 2 smd rect (at -0.65 -1.4625 270) (size 0.4 1.35) (layers F.Cu F.Paste F.Mask) (zone_connect 2))
  (pad 6 thru_hole circle (at -2.5 -1.4625 270) (size 1.45 1.45) (drill 0.85) (layers *.Cu *.Mask) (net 4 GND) (zone_connect 2))
  (pad 6 smd rect (at 1 1.2375 270) (size 1.5 1.9) (layers F.Cu F.Paste F.Mask) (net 4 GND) (zone_connect 2)))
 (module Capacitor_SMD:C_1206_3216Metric (layer F.Cu) (at 189.23 27.21)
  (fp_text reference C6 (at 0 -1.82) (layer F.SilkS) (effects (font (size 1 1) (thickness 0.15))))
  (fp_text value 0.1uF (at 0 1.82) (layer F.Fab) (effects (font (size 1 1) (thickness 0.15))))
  (pad 1 smd roundrect (at -1.4 0) (size 1.25 1.75) (layers F.Cu F.Paste F.Mask) (roundrect_rratio 0.2) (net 1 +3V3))
  (pad 2 smd roundrect (at 1.4 0) (size 1.25 1.75) (layers F.Cu F.Paste F.Mask) (roundrect_rratio 0.2) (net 4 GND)))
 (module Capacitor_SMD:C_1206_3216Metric (layer F.Cu) (at 189.23 42.45)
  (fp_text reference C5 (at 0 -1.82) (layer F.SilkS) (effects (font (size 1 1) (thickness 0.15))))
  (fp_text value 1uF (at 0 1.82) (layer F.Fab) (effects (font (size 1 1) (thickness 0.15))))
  (pad 1 smd roundrect (at -1.4 0) (size 1.25 1.75) (layers F.Cu F.Paste F.Mask) (roundrect_rratio 0.2) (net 3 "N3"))
  (pad 2 smd roundrect (at 1.4 0) (size 1.25 1.75) (layers F.Cu F.Paste F.Mask) (roundrect_rratio 0.2) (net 21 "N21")))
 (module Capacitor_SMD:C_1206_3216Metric (layer F.Cu) (at 189.23 37.37)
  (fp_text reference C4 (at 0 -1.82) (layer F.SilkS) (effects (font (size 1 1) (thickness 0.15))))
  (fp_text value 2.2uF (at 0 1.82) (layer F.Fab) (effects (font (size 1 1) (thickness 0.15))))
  (pad 1 smd roundrect (at -1.4 0) (size 1.25 1.75) (layers F.Cu F.Paste F.Mask) (roundrect_rratio 0.2) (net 2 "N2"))
  (pad 2 smd roundrect (at 1.4 0) (size 1.25 1.75) (layers F.Cu F.Paste F.Mask) (roundrect_rratio 0.2) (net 4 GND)))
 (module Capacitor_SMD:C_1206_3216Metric (layer F.Cu) (at 189.23 32.29)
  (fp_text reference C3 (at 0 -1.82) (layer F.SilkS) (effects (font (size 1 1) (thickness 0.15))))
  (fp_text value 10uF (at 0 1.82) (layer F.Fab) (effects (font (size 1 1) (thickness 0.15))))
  (pad 1 smd roundrect (at -1.4 0) (size 1.25 1.75) (layers F.Cu F.Paste F.Mask) (roundrect_rratio 0.2) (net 1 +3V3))
  (pad 2 smd roundrect (at 1.4 0) (size 1.25 1.75) (layers F.Cu F.Paste F.Mask) (roundrect_rratio 0.2) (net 4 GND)))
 (gr_line (start 82 56) (end 82 19) (layer Edge.Cuts) (width 0.05))
 (gr_line (start 209 56) (end 82 56) (layer Edge.Cuts) (width 0.05))
 (gr_line (start 209 19) (end 209 56) (layer Edge.Cuts) (width 0.05))
 (gr_line (start 82 19) (end 209 19) (layer Edge.Cuts) (width 0.05))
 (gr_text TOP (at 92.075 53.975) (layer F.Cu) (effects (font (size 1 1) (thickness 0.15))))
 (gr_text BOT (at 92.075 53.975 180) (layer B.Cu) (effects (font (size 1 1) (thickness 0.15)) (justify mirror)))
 (segment (start 84.7625 40) (end 83.7625 41) (width 0.4) (layer F.Cu) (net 4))
 (segment (start 84.7625 35) (end 83.7625 34) (width 0.4) (layer F.Cu) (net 4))
 (segment (start 86.4625 35) (end 84.7625 35) (width 0.4) (layer F.Cu) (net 4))
 (segment (start 89.325001 38.850001) (end 86.4625 38.850001) (width 0.2) (layer F.Cu) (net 4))
 (segment (start 90.6 41) (end 90.6 40.125) (width 0.2) (layer F.Cu) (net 4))
 (segment (start 90.6 40.125) (end 89.325001 38.850001) (width 0.2) (layer F.Cu) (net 4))
 (via (at 114.75 48) (size 0.6) (drill 0.3) (layers F.Cu B.Cu) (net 4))
 (segment (start 112.9 48) (end 114.75 48) (width 0.2) (layer F.Cu) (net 4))
 (segment (start 114.75 48) (end 116.745 48) (width 0.2) (layer B.Cu) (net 4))
 (via (at 117 48.255) (size 0.6) (drill 0.3) (layers F.Cu B.Cu) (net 4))
 (segment (start 116.745 48) (end 117 48.255) (width 0.2) (layer B.Cu) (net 4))
 (segment (start 157.5 50.08) (end 157.5 44.92) (width 0.2) (layer B.Cu) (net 4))
 (segment (start 157.5 30.08) (end 157.5 24.92) (width 0.2) (layer B.Cu) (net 4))
 (segment (start 91.973 31) (end 98.273 31) (width 0.2) (layer F.Cu) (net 1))
 (segment (start 109.6 39.75) (end 110.1 40.25) (width 0.2) (layer F.Cu) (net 1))
 (segment (start 103.635 39.75) (end 109.6 39.75) (width 0.2) (layer F.Cu) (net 1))
 (segment (start 110.1 40.25) (end 110.1 44.25) (width 0.2) (layer F.Cu) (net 1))
 (segment (start 110.1 44.25) (end 110.1 48) (width 0.2) (layer F.Cu) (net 1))
 (segment (start 112.10001 46.62499) (end 114.37499 46.62499) (width 0.2) (layer F.Cu) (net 1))
 (segment (start 110.1 48) (end 110.725 48) (width 0.2) (layer F.Cu) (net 1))
 (segment (start 110.725 48) (end 112.10001 46.62499) (width 0.2) (layer F.Cu) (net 1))
 (via (at 114.75 47) (size 0.6) (drill 0.3) (layers F.Cu B.Cu) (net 1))
 (segment (start 114.37499 46.62499) (end 114.75 47) (width 0.2) (layer F.Cu) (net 1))
 (segment (start 116.985 47) (end 117 46.985) (width 0.2) (layer B.Cu) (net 1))
 (segment (start 114.75 47) (end 116.985 47) (width 0.2) (layer B.Cu) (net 1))
 (segment (start 103.635 36) (end 103.635 39.75) (width 0.2) (layer F.Cu) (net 1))
 (segment (start 99.473 31) (end 98.273 31) (width 0.2) (layer F.Cu) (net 1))
 (segment (start 99.51 31) (end 99.473 31) (width 0.2) (layer F.Cu) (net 1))
 (segment (start 103.635 35.125) (end 99.51 31) (width 0.2) (layer F.Cu) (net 1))
 (segment (start 103.635 36) (end 103.635 35.125) (width 0.2) (layer F.Cu) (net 1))
 (segment (start 99.92 31) (end 105.5 25.42) (width 0.2) (layer F.Cu) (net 1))
 (segment (start 98.273 31) (end 99.92 31) (width 0.2) (layer F.Cu) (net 1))
 (segment (start 113.525 40.25) (end 114.75 41.475) (width 0.2) (layer F.Cu) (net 20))
 (segment (start 112.9 40.25) (end 113.525 40.25) (width 0.2) (layer F.Cu) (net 20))
 (via (at 114.75 45.75) (size 0.6) (drill 0.3) (layers F.Cu B.Cu) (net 20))
 (segment (start 114.75 41.475) (end 114.75 45.75) (width 0.2) (layer F.Cu) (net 20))
 (segment (start 116.965 45.75) (end 117 45.715) (width 0.2) (layer B.Cu) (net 20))
 (segment (start 114.75 45.75) (end 116.965 45.75) (width 0.2) (layer B.Cu) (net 20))
 (segment (start 112.9 36.815) (end 112.965 36.75) (width 0.2) (layer F.Cu) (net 20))
 (segment (start 112.9 40.25) (end 112.9 36.815) (width 0.2) (layer F.Cu) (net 20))
 (segment (start 93.4 40.125) (end 93.4 37) (width 0.4) (layer F.Cu) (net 10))
 (segment (start 93.4 41) (end 93.4 40.125) (width 0.4) (layer F.Cu) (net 10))
 (segment (start 93.373 33.3) (end 91.973 33.3) (width 0.4) (layer F.Cu) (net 10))
 (segment (start 93.4 33.327) (end 93.373 33.3) (width 0.4) (layer F.Cu) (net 10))
 (segment (start 93.4 37) (end 93.4 33.327) (width 0.4) (layer F.Cu) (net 10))
 (segment (start 154 49.525) (end 156.475 52) (width 0.2) (layer B.Cu) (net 12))
 (segment (start 154 48.9) (end 154 49.525) (width 0.2) (layer B.Cu) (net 12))
 (segment (start 159.5 51.005) (end 159.5 50.08) (width 0.2) (layer B.Cu) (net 12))
 (segment (start 158.505 52) (end 159.5 51.005) (width 0.2) (layer B.Cu) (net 12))
 (segment (start 156.475 52) (end 158.505 52) (width 0.2) (layer B.Cu) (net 12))
 (segment (start 159.5 50.08) (end 159.5 44.92) (width 0.2) (layer B.Cu) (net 12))
 (segment (start 154 29.775) (end 155.975 31.75) (width 0.2) (layer B.Cu) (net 11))
 (segment (start 154 29.15) (end 154 29.775) (width 0.2) (layer B.Cu) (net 11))
 (segment (start 159.5 31.005) (end 159.5 30.08) (width 0.2) (layer B.Cu) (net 11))
 (segment (start 158.755 31.75) (end 159.5 31.005) (width 0.2) (layer B.Cu) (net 11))
 (segment (start 155.975 31.75) (end 158.755 31.75) (width 0.2) (layer B.Cu) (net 11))
 (segment (start 159.5 30.08) (end 159.5 24.92) (width 0.2) (layer B.Cu) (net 11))
 (segment (start 87.275502 36) (end 87.125503 36.149999) (width 0.2) (layer F.Cu) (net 9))
 (segment (start 90.475 36) (end 87.275502 36) (width 0.2) (layer F.Cu) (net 9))
 (segment (start 90.6 37) (end 90.6 36.125) (width 0.2) (layer F.Cu) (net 9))
 (segment (start 90.6 36.125) (end 90.475 36) (width 0.2) (layer F.Cu) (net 9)))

